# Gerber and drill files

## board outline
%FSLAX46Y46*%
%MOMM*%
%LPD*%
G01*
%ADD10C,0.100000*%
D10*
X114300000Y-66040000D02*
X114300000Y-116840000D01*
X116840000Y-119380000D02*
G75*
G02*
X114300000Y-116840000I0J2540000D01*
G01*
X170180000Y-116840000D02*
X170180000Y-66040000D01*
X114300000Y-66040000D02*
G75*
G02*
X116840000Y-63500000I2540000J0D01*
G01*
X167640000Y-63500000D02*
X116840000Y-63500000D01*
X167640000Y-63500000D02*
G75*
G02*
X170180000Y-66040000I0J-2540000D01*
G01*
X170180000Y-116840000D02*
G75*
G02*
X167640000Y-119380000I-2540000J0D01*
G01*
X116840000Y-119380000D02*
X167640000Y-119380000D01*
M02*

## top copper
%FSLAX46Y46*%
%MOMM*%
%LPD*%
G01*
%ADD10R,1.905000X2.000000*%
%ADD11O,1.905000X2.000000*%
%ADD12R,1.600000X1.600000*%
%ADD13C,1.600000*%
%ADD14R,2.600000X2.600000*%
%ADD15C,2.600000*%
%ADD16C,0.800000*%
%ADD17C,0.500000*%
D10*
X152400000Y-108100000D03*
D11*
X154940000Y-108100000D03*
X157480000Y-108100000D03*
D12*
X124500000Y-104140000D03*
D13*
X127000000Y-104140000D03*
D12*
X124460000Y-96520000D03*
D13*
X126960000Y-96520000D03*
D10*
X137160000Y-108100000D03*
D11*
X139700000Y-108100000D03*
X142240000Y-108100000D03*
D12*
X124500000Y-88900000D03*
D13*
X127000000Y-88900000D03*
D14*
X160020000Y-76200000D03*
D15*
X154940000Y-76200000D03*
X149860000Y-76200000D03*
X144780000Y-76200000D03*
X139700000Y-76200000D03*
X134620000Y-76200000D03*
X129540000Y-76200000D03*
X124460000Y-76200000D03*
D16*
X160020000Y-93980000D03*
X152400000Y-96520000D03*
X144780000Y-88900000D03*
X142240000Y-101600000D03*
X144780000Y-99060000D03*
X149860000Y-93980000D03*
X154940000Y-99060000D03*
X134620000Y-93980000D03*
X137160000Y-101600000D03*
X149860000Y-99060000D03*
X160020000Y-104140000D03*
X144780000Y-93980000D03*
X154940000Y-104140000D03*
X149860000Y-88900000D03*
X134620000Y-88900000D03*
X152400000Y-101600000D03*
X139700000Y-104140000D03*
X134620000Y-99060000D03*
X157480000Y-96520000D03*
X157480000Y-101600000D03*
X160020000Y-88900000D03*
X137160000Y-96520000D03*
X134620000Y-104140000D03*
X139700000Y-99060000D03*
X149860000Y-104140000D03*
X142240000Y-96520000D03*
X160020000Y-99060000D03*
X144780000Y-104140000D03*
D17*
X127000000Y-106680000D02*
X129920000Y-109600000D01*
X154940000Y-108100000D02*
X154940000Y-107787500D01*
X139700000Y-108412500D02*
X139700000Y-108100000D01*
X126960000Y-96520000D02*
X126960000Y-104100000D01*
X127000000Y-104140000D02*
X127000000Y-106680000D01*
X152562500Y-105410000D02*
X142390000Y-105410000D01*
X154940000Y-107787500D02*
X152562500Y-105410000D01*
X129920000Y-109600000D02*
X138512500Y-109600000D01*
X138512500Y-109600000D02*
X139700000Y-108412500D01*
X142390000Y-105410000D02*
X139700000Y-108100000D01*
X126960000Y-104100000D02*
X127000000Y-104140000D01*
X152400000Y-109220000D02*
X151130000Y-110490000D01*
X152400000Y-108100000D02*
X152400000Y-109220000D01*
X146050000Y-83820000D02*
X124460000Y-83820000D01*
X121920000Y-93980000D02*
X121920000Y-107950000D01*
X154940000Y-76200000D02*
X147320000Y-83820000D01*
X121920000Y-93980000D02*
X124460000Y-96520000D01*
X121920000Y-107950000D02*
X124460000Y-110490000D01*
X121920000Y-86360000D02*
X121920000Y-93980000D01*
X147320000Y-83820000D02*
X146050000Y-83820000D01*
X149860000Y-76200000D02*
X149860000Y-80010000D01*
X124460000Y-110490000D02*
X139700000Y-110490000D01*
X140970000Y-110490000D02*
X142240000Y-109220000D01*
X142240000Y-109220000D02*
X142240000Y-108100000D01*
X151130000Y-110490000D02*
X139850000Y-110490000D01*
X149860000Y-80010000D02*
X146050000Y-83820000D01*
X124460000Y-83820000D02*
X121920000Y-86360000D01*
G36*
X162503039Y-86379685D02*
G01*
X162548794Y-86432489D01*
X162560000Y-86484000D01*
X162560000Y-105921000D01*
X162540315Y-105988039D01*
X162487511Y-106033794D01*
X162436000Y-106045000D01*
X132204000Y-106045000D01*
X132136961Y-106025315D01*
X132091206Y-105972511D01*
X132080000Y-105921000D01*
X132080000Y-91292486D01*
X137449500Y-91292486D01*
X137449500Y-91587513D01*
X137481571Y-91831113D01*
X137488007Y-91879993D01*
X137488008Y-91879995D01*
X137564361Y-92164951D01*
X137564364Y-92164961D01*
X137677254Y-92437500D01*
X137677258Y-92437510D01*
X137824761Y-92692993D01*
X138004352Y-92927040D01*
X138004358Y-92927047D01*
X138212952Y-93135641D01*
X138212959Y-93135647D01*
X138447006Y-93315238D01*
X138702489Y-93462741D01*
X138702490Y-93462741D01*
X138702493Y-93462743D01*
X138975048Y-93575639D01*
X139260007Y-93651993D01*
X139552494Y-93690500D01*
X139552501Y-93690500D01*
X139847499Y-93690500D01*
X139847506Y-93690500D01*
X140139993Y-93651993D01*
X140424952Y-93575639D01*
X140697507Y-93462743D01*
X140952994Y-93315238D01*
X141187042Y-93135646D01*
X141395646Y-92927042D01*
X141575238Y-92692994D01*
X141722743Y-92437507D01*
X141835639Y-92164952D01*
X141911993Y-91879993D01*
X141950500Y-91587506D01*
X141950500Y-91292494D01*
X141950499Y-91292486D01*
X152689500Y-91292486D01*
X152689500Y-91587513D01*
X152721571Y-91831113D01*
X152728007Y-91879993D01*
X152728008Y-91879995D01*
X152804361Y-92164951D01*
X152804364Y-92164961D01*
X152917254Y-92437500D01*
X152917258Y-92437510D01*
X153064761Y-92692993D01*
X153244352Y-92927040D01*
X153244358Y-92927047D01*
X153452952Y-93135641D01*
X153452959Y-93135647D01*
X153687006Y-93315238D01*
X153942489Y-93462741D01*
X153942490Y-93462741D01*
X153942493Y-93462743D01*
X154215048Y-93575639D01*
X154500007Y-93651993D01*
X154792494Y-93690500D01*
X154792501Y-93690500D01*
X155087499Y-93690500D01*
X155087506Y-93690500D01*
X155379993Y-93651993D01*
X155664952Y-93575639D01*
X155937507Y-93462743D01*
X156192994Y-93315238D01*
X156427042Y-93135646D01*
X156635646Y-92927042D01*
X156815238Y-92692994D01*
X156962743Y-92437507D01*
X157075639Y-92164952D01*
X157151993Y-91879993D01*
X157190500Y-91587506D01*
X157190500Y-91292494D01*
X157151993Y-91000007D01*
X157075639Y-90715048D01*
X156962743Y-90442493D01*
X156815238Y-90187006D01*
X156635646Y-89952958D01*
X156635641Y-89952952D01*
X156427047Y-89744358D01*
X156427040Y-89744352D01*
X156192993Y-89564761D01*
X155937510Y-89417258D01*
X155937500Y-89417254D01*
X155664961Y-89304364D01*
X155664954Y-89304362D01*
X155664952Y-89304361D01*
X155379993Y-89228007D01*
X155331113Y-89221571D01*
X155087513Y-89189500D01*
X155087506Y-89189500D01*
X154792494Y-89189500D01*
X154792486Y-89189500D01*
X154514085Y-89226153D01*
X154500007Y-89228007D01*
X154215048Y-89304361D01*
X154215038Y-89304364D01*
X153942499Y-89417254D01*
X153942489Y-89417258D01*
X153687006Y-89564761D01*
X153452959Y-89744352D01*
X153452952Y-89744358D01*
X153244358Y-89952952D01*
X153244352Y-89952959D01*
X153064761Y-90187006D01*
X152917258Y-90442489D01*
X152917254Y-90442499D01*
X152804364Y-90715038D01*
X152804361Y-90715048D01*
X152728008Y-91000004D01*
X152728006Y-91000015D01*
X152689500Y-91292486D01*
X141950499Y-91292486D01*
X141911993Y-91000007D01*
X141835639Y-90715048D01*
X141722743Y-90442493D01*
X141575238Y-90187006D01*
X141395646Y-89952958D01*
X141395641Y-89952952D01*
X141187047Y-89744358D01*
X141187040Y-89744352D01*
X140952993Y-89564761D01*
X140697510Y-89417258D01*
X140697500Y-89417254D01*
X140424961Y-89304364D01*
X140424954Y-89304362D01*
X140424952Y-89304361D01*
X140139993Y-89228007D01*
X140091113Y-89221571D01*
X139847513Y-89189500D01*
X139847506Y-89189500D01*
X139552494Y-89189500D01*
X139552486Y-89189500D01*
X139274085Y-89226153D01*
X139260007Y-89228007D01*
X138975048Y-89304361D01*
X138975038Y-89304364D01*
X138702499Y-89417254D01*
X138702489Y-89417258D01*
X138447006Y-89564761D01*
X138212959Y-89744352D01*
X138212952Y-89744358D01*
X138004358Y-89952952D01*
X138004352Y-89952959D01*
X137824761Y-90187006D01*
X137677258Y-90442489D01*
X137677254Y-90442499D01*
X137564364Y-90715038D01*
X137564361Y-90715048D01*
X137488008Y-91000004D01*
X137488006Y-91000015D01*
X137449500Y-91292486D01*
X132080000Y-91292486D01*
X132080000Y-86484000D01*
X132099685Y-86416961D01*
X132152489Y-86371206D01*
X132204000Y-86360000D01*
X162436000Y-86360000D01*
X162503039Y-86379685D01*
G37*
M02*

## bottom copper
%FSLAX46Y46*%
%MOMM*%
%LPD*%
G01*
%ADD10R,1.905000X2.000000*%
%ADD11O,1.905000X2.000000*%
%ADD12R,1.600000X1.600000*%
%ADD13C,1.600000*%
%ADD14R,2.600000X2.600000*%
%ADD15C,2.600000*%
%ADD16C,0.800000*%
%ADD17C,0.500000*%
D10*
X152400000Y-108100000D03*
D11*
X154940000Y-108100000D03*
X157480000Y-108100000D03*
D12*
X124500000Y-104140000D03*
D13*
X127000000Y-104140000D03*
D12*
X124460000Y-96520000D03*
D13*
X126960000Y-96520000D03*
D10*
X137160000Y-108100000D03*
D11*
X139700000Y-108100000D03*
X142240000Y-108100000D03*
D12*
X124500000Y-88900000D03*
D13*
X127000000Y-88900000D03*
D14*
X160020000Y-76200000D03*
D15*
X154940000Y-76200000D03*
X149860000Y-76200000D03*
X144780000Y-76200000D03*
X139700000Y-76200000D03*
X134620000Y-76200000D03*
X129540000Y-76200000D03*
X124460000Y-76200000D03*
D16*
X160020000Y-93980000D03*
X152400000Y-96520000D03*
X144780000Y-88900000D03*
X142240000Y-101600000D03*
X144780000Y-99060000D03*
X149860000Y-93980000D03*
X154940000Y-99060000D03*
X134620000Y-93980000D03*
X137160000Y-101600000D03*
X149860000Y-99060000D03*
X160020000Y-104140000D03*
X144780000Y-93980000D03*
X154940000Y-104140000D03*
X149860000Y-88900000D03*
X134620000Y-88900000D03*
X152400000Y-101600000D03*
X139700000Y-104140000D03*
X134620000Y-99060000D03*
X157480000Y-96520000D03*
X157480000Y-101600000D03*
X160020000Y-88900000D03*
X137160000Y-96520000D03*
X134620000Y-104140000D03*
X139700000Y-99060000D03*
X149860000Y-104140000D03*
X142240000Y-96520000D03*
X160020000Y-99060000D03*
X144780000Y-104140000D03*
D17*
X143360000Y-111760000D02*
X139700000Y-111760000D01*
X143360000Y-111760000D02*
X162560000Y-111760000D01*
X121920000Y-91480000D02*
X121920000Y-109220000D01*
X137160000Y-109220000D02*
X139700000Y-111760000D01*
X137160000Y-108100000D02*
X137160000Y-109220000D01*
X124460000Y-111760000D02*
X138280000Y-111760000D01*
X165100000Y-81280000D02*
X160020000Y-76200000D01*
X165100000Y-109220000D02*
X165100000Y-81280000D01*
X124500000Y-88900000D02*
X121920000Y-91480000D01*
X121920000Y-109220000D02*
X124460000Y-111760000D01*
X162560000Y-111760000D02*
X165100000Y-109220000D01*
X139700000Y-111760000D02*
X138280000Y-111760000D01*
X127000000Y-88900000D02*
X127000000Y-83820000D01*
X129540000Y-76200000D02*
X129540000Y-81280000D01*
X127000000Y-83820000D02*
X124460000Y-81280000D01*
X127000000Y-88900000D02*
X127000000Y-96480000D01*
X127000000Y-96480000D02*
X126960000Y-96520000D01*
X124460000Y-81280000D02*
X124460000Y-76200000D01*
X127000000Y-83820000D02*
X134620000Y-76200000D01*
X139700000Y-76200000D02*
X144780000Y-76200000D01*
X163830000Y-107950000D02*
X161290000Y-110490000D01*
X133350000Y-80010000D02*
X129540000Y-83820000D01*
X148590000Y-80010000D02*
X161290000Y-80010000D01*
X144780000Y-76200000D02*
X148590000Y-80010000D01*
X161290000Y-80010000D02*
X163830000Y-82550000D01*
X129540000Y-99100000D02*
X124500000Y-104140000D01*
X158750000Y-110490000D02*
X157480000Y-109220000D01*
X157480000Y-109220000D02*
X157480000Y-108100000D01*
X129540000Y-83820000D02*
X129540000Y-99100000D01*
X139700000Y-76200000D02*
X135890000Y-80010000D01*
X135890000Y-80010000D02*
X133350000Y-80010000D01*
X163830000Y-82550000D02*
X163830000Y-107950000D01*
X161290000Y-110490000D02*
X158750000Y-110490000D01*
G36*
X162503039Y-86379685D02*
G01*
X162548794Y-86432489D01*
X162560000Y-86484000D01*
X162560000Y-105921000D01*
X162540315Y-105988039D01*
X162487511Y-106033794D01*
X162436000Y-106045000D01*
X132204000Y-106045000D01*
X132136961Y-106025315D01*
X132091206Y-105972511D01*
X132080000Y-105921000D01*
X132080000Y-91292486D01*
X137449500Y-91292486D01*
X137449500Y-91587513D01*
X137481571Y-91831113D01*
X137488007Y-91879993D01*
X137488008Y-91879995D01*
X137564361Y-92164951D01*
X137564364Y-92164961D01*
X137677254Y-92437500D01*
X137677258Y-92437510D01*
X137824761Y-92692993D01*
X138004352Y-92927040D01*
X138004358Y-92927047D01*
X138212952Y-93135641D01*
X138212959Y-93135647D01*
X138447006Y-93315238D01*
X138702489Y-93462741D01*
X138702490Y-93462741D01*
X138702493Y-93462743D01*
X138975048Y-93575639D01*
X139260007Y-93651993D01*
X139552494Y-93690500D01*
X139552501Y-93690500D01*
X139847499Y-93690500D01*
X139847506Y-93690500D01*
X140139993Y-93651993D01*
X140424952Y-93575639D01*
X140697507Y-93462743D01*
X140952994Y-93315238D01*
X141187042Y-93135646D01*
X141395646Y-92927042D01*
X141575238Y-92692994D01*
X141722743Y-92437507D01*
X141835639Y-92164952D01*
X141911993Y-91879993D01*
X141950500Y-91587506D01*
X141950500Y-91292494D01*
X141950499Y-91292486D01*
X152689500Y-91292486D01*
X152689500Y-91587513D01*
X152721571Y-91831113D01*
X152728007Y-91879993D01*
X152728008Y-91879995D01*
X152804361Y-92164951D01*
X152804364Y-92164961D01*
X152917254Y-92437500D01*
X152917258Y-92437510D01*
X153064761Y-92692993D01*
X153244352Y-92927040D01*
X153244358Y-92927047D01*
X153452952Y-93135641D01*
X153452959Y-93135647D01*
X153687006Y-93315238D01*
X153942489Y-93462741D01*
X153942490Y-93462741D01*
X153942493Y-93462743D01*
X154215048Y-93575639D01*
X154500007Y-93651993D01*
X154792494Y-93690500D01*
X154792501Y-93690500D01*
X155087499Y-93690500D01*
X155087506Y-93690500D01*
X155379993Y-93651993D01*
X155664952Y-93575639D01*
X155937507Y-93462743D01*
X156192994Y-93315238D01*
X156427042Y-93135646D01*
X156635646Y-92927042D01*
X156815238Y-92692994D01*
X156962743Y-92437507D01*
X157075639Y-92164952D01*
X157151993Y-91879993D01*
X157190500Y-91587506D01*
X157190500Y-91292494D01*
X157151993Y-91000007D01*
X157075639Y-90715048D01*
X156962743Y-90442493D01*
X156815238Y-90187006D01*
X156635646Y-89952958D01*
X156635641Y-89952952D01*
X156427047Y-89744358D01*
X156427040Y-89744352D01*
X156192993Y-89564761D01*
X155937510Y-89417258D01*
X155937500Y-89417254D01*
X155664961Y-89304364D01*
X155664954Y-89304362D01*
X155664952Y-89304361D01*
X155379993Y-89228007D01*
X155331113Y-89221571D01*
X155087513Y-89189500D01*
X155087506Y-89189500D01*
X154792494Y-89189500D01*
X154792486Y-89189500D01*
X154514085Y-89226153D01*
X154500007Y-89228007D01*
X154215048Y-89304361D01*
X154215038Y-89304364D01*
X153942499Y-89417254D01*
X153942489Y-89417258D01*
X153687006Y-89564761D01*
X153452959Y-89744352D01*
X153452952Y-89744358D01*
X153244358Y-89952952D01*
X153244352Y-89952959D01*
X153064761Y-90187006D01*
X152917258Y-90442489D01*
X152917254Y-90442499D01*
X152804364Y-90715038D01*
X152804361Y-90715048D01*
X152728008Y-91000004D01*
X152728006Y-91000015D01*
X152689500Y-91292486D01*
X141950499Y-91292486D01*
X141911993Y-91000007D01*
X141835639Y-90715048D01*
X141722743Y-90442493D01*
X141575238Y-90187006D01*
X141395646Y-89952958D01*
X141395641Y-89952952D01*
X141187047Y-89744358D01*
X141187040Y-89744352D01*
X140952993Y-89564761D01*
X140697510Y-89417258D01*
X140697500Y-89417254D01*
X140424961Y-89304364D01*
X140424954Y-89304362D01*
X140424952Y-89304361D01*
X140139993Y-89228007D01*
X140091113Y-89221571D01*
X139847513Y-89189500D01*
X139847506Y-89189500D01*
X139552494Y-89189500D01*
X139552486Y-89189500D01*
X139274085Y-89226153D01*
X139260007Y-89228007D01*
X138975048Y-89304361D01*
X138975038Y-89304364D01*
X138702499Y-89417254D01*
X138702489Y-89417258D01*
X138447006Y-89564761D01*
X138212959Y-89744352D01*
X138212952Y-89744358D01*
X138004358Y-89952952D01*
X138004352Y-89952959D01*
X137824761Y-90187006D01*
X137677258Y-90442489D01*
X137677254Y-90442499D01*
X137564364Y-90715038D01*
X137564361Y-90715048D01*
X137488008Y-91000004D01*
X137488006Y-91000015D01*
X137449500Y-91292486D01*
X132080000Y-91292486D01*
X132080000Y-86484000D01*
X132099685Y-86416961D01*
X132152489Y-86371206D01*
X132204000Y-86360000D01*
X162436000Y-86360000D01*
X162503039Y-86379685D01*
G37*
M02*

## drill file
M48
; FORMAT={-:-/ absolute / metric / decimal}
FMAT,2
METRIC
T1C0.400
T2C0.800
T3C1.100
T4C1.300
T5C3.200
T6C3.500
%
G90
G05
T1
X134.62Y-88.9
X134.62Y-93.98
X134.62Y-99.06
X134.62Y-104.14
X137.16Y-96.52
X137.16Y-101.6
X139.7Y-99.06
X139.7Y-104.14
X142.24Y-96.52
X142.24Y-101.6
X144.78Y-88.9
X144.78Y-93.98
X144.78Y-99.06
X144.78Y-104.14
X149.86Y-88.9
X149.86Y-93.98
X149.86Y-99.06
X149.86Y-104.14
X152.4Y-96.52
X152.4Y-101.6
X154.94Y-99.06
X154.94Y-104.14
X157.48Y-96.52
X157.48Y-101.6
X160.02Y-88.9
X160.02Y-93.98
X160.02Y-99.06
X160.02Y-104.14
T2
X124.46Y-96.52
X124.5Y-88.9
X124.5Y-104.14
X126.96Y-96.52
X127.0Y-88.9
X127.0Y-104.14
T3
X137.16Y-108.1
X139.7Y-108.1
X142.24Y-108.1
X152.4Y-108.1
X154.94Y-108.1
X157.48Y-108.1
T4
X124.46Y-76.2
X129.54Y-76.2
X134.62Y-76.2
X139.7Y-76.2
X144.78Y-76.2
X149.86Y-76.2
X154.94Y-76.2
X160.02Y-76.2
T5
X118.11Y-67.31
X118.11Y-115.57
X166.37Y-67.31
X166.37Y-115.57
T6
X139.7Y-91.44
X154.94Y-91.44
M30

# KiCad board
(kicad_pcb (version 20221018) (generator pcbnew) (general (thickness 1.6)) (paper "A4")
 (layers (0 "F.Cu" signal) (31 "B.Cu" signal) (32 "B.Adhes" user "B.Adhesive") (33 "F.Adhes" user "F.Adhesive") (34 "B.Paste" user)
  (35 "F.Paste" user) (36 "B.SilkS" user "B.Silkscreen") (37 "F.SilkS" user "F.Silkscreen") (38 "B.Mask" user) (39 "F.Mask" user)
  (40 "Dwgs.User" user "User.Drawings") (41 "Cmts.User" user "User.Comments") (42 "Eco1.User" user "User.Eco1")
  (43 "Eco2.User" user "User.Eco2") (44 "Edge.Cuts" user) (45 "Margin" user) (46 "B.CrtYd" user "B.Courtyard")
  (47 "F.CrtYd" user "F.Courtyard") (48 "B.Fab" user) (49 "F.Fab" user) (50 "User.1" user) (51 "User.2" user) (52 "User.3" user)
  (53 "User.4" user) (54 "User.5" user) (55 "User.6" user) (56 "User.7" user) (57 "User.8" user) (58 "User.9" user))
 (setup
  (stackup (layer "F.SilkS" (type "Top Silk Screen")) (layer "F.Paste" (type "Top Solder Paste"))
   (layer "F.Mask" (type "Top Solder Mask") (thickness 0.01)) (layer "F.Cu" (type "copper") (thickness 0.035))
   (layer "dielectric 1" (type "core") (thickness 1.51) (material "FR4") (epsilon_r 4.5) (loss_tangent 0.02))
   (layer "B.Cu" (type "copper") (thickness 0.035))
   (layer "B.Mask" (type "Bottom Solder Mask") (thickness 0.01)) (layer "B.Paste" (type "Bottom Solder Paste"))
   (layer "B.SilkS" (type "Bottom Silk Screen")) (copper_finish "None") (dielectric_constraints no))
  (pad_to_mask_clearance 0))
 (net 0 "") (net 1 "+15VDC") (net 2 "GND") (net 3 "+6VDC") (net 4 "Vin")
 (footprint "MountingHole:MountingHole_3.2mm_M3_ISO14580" (layer "F.Cu") (at 166.37 67.31)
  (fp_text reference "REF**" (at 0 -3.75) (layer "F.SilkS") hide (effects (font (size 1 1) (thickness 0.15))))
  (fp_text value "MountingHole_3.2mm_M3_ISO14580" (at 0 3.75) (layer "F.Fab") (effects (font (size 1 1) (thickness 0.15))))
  (pad "" np_thru_hole circle (at 0 0) (size 3.2 3.2) (drill 3.2) (layers "*.Cu" "*.Mask")))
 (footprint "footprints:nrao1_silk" (layer "F.Cu") (at 127 113.03)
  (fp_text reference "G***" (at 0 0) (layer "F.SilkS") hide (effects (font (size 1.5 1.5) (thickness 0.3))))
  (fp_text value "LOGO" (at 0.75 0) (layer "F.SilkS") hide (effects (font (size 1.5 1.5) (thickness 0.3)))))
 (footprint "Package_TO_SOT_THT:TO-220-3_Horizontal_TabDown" (layer "F.Cu") (at 152.4 108.1)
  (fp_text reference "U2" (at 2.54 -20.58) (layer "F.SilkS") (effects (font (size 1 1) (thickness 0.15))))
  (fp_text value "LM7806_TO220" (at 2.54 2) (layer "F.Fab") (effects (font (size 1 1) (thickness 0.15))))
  (pad "" np_thru_hole oval (at 2.54 -16.66) (size 3.5 3.5) (drill 3.5) (layers "*.Cu" "*.Mask"))
  (pad "1" thru_hole rect (at 0 0) (size 1.905 2) (drill 1.1) (layers "*.Cu" "*.Mask") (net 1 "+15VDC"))
  (pad "2" thru_hole oval (at 2.54 0) (size 1.905 2) (drill 1.1) (layers "*.Cu" "*.Mask") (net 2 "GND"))
  (pad "3" thru_hole oval (at 5.08 0) (size 1.905 2) (drill 1.1) (layers "*.Cu" "*.Mask") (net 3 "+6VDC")))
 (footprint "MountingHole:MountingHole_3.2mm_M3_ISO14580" (layer "F.Cu") (at 118.11 67.31)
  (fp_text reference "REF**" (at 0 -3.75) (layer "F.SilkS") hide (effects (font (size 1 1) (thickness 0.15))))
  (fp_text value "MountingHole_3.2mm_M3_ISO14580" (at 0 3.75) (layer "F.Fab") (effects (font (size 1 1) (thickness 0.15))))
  (pad "" np_thru_hole circle (at 0 0) (size 3.2 3.2) (drill 3.2) (layers "*.Cu" "*.Mask")))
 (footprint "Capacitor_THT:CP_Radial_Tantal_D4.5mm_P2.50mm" (layer "F.Cu") (at 124.5 104.14)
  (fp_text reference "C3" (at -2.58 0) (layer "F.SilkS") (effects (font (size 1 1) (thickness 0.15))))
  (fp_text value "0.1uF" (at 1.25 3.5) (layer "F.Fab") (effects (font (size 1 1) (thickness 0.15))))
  (pad "1" thru_hole rect (at 0 0) (size 1.6 1.6) (drill 0.8) (layers "*.Cu" "*.Mask") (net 3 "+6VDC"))
  (pad "2" thru_hole circle (at 2.5 0) (size 1.6 1.6) (drill 0.8) (layers "*.Cu" "*.Mask") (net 2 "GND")))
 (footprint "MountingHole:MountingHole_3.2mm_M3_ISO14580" (layer "F.Cu") (at 118.11 115.57)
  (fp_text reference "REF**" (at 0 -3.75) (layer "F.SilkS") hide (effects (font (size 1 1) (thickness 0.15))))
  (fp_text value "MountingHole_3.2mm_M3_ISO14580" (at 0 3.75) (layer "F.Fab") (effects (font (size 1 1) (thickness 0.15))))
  (pad "" np_thru_hole circle (at 0 0) (size 3.2 3.2) (drill 3.2) (layers "*.Cu" "*.Mask")))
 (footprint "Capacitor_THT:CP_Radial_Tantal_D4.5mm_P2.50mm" (layer "F.Cu") (at 124.46 96.52)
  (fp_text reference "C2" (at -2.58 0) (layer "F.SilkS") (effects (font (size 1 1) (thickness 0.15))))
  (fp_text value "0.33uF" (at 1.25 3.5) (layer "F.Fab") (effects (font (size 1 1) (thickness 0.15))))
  (pad "1" thru_hole rect (at 0 0) (size 1.6 1.6) (drill 0.8) (layers "*.Cu" "*.Mask") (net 1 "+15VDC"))
  (pad "2" thru_hole circle (at 2.5 0) (size 1.6 1.6) (drill 0.8) (layers "*.Cu" "*.Mask") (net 2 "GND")))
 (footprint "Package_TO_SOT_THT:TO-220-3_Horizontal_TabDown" (layer "F.Cu") (at 137.16 108.1)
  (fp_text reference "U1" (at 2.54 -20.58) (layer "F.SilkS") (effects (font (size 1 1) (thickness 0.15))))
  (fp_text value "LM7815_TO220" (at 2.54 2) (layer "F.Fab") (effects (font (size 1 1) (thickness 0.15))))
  (pad "" np_thru_hole oval (at 2.54 -16.66) (size 3.5 3.5) (drill 3.5) (layers "*.Cu" "*.Mask"))
  (pad "1" thru_hole rect (at 0 0) (size 1.905 2) (drill 1.1) (layers "*.Cu" "*.Mask") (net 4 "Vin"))
  (pad "2" thru_hole oval (at 2.54 0) (size 1.905 2) (drill 1.1) (layers "*.Cu" "*.Mask") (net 2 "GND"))
  (pad "3" thru_hole oval (at 5.08 0) (size 1.905 2) (drill 1.1) (layers "*.Cu" "*.Mask") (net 1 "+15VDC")))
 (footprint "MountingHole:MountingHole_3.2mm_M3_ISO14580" (layer "F.Cu") (at 166.37 115.57)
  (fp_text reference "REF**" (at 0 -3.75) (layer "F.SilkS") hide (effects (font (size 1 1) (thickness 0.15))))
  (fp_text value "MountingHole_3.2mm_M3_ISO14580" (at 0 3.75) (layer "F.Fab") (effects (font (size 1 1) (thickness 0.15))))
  (pad "" np_thru_hole circle (at 0 0) (size 3.2 3.2) (drill 3.2) (layers "*.Cu" "*.Mask")))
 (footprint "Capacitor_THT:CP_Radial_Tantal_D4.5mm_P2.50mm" (layer "F.Cu") (at 124.5 88.9)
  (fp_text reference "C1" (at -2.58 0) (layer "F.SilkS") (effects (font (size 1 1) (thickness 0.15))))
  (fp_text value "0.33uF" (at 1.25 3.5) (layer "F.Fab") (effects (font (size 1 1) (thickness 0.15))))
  (pad "1" thru_hole rect (at 0 0) (size 1.6 1.6) (drill 0.8) (layers "*.Cu" "*.Mask") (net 4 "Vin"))
  (pad "2" thru_hole circle (at 2.5 0) (size 1.6 1.6) (drill 0.8) (layers "*.Cu" "*.Mask") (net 2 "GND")))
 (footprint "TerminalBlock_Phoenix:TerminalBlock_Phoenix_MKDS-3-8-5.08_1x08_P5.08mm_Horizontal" (layer "F.Cu") (at 160.02 76.2 180)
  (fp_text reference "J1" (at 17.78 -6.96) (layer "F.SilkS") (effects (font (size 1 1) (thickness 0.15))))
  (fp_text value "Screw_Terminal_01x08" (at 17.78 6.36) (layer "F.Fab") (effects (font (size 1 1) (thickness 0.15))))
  (pad "1" thru_hole rect (at 0 0 180) (size 2.6 2.6) (drill 1.3) (layers "*.Cu" "*.Mask") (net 4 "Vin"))
  (pad "2" thru_hole circle (at 5.08 0 180) (size 2.6 2.6) (drill 1.3) (layers "*.Cu" "*.Mask") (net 1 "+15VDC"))
  (pad "3" thru_hole circle (at 10.16 0 180) (size 2.6 2.6) (drill 1.3) (layers "*.Cu" "*.Mask") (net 1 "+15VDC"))
  (pad "4" thru_hole circle (at 15.24 0 180) (size 2.6 2.6) (drill 1.3) (layers "*.Cu" "*.Mask") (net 3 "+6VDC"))
  (pad "5" thru_hole circle (at 20.32 0 180) (size 2.6 2.6) (drill 1.3) (layers "*.Cu" "*.Mask") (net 3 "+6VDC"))
  (pad "6" thru_hole circle (at 25.4 0 180) (size 2.6 2.6) (drill 1.3) (layers "*.Cu" "*.Mask") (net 2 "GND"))
  (pad "7" thru_hole circle (at 30.48 0 180) (size 2.6 2.6) (drill 1.3) (layers "*.Cu" "*.Mask") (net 2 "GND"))
  (pad "8" thru_hole circle (at 35.56 0 180) (size 2.6 2.6) (drill 1.3) (layers "*.Cu" "*.Mask") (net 2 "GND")))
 (gr_line (start 114.3 66.04) (end 114.3 116.84) (stroke (width 0.1) (type default)) (layer "Edge.Cuts"))
 (gr_arc (start 116.84 119.38) (mid 115.043949 118.636051) (end 114.3 116.84) (stroke (width 0.1) (type default)) (layer "Edge.Cuts"))
 (gr_line (start 170.18 116.84) (end 170.18 66.04) (stroke (width 0.1) (type default)) (layer "Edge.Cuts"))
 (gr_arc (start 114.3 66.04) (mid 115.043949 64.243949) (end 116.84 63.5) (stroke (width 0.1) (type default)) (layer "Edge.Cuts"))
 (gr_line (start 167.64 63.5) (end 116.84 63.5) (stroke (width 0.1) (type default)) (layer "Edge.Cuts"))
 (gr_arc (start 167.64 63.5) (mid 169.436051 64.243949) (end 170.18 66.04) (stroke (width 0.1) (type default)) (layer "Edge.Cuts"))
 (gr_arc (start 170.18 116.84) (mid 169.436051 118.636051) (end 167.64 119.38) (stroke (width 0.1) (type default)) (layer "Edge.Cuts"))
 (gr_line (start 116.84 119.38) (end 167.64 119.38) (stroke (width 0.1) (type default)) (layer "Edge.Cuts"))
 (segment (start 143.36 111.76) (end 139.7 111.76) (width 0.5) (layer "B.Cu") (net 4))
 (segment (start 143.36 111.76) (end 162.56 111.76) (width 0.5) (layer "B.Cu") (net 4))
 (segment (start 121.92 91.48) (end 121.92 109.22) (width 0.5) (layer "B.Cu") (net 4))
 (segment (start 137.16 109.22) (end 139.7 111.76) (width 0.5) (layer "B.Cu") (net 4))
 (segment (start 137.16 108.1) (end 137.16 109.22) (width 0.5) (layer "B.Cu") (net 4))
 (segment (start 124.46 111.76) (end 138.28 111.76) (width 0.5) (layer "B.Cu") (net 4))
 (segment (start 165.1 81.28) (end 160.02 76.2) (width 0.5) (layer "B.Cu") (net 4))
 (segment (start 165.1 109.22) (end 165.1 81.28) (width 0.5) (layer "B.Cu") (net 4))
 (segment (start 124.5 88.9) (end 121.92 91.48) (width 0.5) (layer "B.Cu") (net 4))
 (segment (start 121.92 109.22) (end 124.46 111.76) (width 0.5) (layer "B.Cu") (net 4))
 (segment (start 162.56 111.76) (end 165.1 109.22) (width 0.5) (layer "B.Cu") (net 4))
 (segment (start 139.7 111.76) (end 138.28 111.76) (width 0.5) (layer "B.Cu") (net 4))
 (segment (start 127 106.68) (end 129.92 109.6) (width 0.5) (layer "F.Cu") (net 2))
 (segment (start 154.94 108.1) (end 154.94 107.7875) (width 0.5) (layer "F.Cu") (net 2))
 (segment (start 139.7 108.4125) (end 139.7 108.1) (width 0.5) (layer "F.Cu") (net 2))
 (segment (start 126.96 96.52) (end 126.96 104.1) (width 0.5) (layer "F.Cu") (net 2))
 (segment (start 127 104.14) (end 127 106.68) (width 0.5) (layer "F.Cu") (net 2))
 (segment (start 152.5625 105.41) (end 142.39 105.41) (width 0.5) (layer "F.Cu") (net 2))
 (segment (start 154.94 107.7875) (end 152.5625 105.41) (width 0.5) (layer "F.Cu") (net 2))
 (segment (start 129.92 109.6) (end 138.5125 109.6) (width 0.5) (layer "F.Cu") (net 2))
 (segment (start 138.5125 109.6) (end 139.7 108.4125) (width 0.5) (layer "F.Cu") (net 2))
 (segment (start 142.39 105.41) (end 139.7 108.1) (width 0.5) (layer "F.Cu") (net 2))
 (segment (start 126.96 104.1) (end 127 104.14) (width 0.5) (layer "F.Cu") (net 2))
 (via (at 160.02 93.98) (size 0.8) (drill 0.4) (layers "F.Cu" "B.Cu") (free) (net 2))
 (via (at 152.4 96.52) (size 0.8) (drill 0.4) (layers "F.Cu" "B.Cu") (free) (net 2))
 (via (at 144.78 88.9) (size 0.8) (drill 0.4) (layers "F.Cu" "B.Cu") (free) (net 2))
 (via (at 142.24 101.6) (size 0.8) (drill 0.4) (layers "F.Cu" "B.Cu") (free) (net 2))
 (via (at 144.78 99.06) (size 0.8) (drill 0.4) (layers "F.Cu" "B.Cu") (free) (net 2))
 (via (at 149.86 93.98) (size 0.8) (drill 0.4) (layers "F.Cu" "B.Cu") (free) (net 2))
 (via (at 154.94 99.06) (size 0.8) (drill 0.4) (layers "F.Cu" "B.Cu") (free) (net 2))
 (via (at 134.62 93.98) (size 0.8) (drill 0.4) (layers "F.Cu" "B.Cu") (free) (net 2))
 (via (at 137.16 101.6) (size 0.8) (drill 0.4) (layers "F.Cu" "B.Cu") (free) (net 2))
 (via (at 149.86 99.06) (size 0.8) (drill 0.4) (layers "F.Cu" "B.Cu") (free) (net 2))
 (via (at 160.02 104.14) (size 0.8) (drill 0.4) (layers "F.Cu" "B.Cu") (free) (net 2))
 (via (at 144.78 93.98) (size 0.8) (drill 0.4) (layers "F.Cu" "B.Cu") (free) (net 2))
 (via (at 154.94 104.14) (size 0.8) (drill 0.4) (layers "F.Cu" "B.Cu") (free) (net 2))
 (via (at 149.86 88.9) (size 0.8) (drill 0.4) (layers "F.Cu" "B.Cu") (free) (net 2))
 (via (at 134.62 88.9) (size 0.8) (drill 0.4) (layers "F.Cu" "B.Cu") (free) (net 2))
 (via (at 152.4 101.6) (size 0.8) (drill 0.4) (layers "F.Cu" "B.Cu") (free) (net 2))
 (via (at 139.7 104.14) (size 0.8) (drill 0.4) (layers "F.Cu" "B.Cu") (free) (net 2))
 (via (at 134.62 99.06) (size 0.8) (drill 0.4) (layers "F.Cu" "B.Cu") (free) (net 2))
 (via (at 157.48 96.52) (size 0.8) (drill 0.4) (layers "F.Cu" "B.Cu") (free) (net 2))
 (via (at 157.48 101.6) (size 0.8) (drill 0.4) (layers "F.Cu" "B.Cu") (free) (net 2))
 (via (at 160.02 88.9) (size 0.8) (drill 0.4) (layers "F.Cu" "B.Cu") (free) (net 2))
 (via (at 137.16 96.52) (size 0.8) (drill 0.4) (layers "F.Cu" "B.Cu") (free) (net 2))
 (via (at 134.62 104.14) (size 0.8) (drill 0.4) (layers "F.Cu" "B.Cu") (free) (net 2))
 (via (at 139.7 99.06) (size 0.8) (drill 0.4) (layers "F.Cu" "B.Cu") (free) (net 2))
 (via (at 149.86 104.14) (size 0.8) (drill 0.4) (layers "F.Cu" "B.Cu") (free) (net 2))
 (via (at 142.24 96.52) (size 0.8) (drill 0.4) (layers "F.Cu" "B.Cu") (free) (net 2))
 (via (at 160.02 99.06) (size 0.8) (drill 0.4) (layers "F.Cu" "B.Cu") (free) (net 2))
 (via (at 144.78 104.14) (size 0.8) (drill 0.4) (layers "F.Cu" "B.Cu") (free) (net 2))
 (segment (start 127 88.9) (end 127 83.82) (width 0.5) (layer "B.Cu") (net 2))
 (segment (start 129.54 76.2) (end 129.54 81.28) (width 0.5) (layer "B.Cu") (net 2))
 (segment (start 127 83.82) (end 124.46 81.28) (width 0.5) (layer "B.Cu") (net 2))
 (segment (start 127 88.9) (end 127 96.48) (width 0.5) (layer "B.Cu") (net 2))
 (segment (start 127 96.48) (end 126.96 96.52) (width 0.5) (layer "B.Cu") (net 2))
 (segment (start 124.46 81.28) (end 124.46 76.2) (width 0.5) (layer "B.Cu") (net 2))
 (segment (start 127 83.82) (end 134.62 76.2) (width 0.5) (layer "B.Cu") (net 2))
 (segment (start 152.4 109.22) (end 151.13 110.49) (width 0.5) (layer "F.Cu") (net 1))
 (segment (start 152.4 108.1) (end 152.4 109.22) (width 0.5) (layer "F.Cu") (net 1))
 (segment (start 146.05 83.82) (end 124.46 83.82) (width 0.5) (layer "F.Cu") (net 1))
 (segment (start 121.92 93.98) (end 121.92 107.95) (width 0.5) (layer "F.Cu") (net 1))
 (segment (start 154.94 76.2) (end 147.32 83.82) (width 0.5) (layer "F.Cu") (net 1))
 (segment (start 121.92 93.98) (end 124.46 96.52) (width 0.5) (layer "F.Cu") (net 1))
 (segment (start 121.92 107.95) (end 124.46 110.49) (width 0.5) (layer "F.Cu") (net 1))
 (segment (start 121.92 86.36) (end 121.92 93.98) (width 0.5) (layer "F.Cu") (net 1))
 (segment (start 147.32 83.82) (end 146.05 83.82) (width 0.5) (layer "F.Cu") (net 1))
 (segment (start 149.86 76.2) (end 149.86 80.01) (width 0.5) (layer "F.Cu") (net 1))
 (segment (start 124.46 110.49) (end 139.7 110.49) (width 0.5) (layer "F.Cu") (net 1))
 (segment (start 140.97 110.49) (end 142.24 109.22) (width 0.5) (layer "F.Cu") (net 1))
 (segment (start 142.24 109.22) (end 142.24 108.1) (width 0.5) (layer "F.Cu") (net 1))
 (segment (start 151.13 110.49) (end 139.85 110.49) (width 0.5) (layer "F.Cu") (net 1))
 (segment (start 149.86 80.01) (end 146.05 83.82) (width 0.5) (layer "F.Cu") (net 1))
 (segment (start 124.46 83.82) (end 121.92 86.36) (width 0.5) (layer "F.Cu") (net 1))
 (segment (start 139.7 76.2) (end 144.78 76.2) (width 0.5) (layer "B.Cu") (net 3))
 (segment (start 163.83 107.95) (end 161.29 110.49) (width 0.5) (layer "B.Cu") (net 3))
 (segment (start 133.35 80.01) (end 129.54 83.82) (width 0.5) (layer "B.Cu") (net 3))
 (segment (start 148.59 80.01) (end 161.29 80.01) (width 0.5) (layer "B.Cu") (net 3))
 (segment (start 144.78 76.2) (end 148.59 80.01) (width 0.5) (layer "B.Cu") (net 3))
 (segment (start 161.29 80.01) (end 163.83 82.55) (width 0.5) (layer "B.Cu") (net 3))
 (segment (start 129.54 99.1) (end 124.5 104.14) (width 0.5) (layer "B.Cu") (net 3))
 (segment (start 158.75 110.49) (end 157.48 109.22) (width 0.5) (layer "B.Cu") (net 3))
 (segment (start 157.48 109.22) (end 157.48 108.1) (width 0.5) (layer "B.Cu") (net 3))
 (segment (start 129.54 83.82) (end 129.54 99.1) (width 0.5) (layer "B.Cu") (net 3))
 (segment (start 139.7 76.2) (end 135.89 80.01) (width 0.5) (layer "B.Cu") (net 3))
 (segment (start 135.89 80.01) (end 133.35 80.01) (width 0.5) (layer "B.Cu") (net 3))
 (segment (start 163.83 82.55) (end 163.83 107.95) (width 0.5) (layer "B.Cu") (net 3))
 (segment (start 161.29 110.49) (end 158.75 110.49) (width 0.5) (layer "B.Cu") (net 3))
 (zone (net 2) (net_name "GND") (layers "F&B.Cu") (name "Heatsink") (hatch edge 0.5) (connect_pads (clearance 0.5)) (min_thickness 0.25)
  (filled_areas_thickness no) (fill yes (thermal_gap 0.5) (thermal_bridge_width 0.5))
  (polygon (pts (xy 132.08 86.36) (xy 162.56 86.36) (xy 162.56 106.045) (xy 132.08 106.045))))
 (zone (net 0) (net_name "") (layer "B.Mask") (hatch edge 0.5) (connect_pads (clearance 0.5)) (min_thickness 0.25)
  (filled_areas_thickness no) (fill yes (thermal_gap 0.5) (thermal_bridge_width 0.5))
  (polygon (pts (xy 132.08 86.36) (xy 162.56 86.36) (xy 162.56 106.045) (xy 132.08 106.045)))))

